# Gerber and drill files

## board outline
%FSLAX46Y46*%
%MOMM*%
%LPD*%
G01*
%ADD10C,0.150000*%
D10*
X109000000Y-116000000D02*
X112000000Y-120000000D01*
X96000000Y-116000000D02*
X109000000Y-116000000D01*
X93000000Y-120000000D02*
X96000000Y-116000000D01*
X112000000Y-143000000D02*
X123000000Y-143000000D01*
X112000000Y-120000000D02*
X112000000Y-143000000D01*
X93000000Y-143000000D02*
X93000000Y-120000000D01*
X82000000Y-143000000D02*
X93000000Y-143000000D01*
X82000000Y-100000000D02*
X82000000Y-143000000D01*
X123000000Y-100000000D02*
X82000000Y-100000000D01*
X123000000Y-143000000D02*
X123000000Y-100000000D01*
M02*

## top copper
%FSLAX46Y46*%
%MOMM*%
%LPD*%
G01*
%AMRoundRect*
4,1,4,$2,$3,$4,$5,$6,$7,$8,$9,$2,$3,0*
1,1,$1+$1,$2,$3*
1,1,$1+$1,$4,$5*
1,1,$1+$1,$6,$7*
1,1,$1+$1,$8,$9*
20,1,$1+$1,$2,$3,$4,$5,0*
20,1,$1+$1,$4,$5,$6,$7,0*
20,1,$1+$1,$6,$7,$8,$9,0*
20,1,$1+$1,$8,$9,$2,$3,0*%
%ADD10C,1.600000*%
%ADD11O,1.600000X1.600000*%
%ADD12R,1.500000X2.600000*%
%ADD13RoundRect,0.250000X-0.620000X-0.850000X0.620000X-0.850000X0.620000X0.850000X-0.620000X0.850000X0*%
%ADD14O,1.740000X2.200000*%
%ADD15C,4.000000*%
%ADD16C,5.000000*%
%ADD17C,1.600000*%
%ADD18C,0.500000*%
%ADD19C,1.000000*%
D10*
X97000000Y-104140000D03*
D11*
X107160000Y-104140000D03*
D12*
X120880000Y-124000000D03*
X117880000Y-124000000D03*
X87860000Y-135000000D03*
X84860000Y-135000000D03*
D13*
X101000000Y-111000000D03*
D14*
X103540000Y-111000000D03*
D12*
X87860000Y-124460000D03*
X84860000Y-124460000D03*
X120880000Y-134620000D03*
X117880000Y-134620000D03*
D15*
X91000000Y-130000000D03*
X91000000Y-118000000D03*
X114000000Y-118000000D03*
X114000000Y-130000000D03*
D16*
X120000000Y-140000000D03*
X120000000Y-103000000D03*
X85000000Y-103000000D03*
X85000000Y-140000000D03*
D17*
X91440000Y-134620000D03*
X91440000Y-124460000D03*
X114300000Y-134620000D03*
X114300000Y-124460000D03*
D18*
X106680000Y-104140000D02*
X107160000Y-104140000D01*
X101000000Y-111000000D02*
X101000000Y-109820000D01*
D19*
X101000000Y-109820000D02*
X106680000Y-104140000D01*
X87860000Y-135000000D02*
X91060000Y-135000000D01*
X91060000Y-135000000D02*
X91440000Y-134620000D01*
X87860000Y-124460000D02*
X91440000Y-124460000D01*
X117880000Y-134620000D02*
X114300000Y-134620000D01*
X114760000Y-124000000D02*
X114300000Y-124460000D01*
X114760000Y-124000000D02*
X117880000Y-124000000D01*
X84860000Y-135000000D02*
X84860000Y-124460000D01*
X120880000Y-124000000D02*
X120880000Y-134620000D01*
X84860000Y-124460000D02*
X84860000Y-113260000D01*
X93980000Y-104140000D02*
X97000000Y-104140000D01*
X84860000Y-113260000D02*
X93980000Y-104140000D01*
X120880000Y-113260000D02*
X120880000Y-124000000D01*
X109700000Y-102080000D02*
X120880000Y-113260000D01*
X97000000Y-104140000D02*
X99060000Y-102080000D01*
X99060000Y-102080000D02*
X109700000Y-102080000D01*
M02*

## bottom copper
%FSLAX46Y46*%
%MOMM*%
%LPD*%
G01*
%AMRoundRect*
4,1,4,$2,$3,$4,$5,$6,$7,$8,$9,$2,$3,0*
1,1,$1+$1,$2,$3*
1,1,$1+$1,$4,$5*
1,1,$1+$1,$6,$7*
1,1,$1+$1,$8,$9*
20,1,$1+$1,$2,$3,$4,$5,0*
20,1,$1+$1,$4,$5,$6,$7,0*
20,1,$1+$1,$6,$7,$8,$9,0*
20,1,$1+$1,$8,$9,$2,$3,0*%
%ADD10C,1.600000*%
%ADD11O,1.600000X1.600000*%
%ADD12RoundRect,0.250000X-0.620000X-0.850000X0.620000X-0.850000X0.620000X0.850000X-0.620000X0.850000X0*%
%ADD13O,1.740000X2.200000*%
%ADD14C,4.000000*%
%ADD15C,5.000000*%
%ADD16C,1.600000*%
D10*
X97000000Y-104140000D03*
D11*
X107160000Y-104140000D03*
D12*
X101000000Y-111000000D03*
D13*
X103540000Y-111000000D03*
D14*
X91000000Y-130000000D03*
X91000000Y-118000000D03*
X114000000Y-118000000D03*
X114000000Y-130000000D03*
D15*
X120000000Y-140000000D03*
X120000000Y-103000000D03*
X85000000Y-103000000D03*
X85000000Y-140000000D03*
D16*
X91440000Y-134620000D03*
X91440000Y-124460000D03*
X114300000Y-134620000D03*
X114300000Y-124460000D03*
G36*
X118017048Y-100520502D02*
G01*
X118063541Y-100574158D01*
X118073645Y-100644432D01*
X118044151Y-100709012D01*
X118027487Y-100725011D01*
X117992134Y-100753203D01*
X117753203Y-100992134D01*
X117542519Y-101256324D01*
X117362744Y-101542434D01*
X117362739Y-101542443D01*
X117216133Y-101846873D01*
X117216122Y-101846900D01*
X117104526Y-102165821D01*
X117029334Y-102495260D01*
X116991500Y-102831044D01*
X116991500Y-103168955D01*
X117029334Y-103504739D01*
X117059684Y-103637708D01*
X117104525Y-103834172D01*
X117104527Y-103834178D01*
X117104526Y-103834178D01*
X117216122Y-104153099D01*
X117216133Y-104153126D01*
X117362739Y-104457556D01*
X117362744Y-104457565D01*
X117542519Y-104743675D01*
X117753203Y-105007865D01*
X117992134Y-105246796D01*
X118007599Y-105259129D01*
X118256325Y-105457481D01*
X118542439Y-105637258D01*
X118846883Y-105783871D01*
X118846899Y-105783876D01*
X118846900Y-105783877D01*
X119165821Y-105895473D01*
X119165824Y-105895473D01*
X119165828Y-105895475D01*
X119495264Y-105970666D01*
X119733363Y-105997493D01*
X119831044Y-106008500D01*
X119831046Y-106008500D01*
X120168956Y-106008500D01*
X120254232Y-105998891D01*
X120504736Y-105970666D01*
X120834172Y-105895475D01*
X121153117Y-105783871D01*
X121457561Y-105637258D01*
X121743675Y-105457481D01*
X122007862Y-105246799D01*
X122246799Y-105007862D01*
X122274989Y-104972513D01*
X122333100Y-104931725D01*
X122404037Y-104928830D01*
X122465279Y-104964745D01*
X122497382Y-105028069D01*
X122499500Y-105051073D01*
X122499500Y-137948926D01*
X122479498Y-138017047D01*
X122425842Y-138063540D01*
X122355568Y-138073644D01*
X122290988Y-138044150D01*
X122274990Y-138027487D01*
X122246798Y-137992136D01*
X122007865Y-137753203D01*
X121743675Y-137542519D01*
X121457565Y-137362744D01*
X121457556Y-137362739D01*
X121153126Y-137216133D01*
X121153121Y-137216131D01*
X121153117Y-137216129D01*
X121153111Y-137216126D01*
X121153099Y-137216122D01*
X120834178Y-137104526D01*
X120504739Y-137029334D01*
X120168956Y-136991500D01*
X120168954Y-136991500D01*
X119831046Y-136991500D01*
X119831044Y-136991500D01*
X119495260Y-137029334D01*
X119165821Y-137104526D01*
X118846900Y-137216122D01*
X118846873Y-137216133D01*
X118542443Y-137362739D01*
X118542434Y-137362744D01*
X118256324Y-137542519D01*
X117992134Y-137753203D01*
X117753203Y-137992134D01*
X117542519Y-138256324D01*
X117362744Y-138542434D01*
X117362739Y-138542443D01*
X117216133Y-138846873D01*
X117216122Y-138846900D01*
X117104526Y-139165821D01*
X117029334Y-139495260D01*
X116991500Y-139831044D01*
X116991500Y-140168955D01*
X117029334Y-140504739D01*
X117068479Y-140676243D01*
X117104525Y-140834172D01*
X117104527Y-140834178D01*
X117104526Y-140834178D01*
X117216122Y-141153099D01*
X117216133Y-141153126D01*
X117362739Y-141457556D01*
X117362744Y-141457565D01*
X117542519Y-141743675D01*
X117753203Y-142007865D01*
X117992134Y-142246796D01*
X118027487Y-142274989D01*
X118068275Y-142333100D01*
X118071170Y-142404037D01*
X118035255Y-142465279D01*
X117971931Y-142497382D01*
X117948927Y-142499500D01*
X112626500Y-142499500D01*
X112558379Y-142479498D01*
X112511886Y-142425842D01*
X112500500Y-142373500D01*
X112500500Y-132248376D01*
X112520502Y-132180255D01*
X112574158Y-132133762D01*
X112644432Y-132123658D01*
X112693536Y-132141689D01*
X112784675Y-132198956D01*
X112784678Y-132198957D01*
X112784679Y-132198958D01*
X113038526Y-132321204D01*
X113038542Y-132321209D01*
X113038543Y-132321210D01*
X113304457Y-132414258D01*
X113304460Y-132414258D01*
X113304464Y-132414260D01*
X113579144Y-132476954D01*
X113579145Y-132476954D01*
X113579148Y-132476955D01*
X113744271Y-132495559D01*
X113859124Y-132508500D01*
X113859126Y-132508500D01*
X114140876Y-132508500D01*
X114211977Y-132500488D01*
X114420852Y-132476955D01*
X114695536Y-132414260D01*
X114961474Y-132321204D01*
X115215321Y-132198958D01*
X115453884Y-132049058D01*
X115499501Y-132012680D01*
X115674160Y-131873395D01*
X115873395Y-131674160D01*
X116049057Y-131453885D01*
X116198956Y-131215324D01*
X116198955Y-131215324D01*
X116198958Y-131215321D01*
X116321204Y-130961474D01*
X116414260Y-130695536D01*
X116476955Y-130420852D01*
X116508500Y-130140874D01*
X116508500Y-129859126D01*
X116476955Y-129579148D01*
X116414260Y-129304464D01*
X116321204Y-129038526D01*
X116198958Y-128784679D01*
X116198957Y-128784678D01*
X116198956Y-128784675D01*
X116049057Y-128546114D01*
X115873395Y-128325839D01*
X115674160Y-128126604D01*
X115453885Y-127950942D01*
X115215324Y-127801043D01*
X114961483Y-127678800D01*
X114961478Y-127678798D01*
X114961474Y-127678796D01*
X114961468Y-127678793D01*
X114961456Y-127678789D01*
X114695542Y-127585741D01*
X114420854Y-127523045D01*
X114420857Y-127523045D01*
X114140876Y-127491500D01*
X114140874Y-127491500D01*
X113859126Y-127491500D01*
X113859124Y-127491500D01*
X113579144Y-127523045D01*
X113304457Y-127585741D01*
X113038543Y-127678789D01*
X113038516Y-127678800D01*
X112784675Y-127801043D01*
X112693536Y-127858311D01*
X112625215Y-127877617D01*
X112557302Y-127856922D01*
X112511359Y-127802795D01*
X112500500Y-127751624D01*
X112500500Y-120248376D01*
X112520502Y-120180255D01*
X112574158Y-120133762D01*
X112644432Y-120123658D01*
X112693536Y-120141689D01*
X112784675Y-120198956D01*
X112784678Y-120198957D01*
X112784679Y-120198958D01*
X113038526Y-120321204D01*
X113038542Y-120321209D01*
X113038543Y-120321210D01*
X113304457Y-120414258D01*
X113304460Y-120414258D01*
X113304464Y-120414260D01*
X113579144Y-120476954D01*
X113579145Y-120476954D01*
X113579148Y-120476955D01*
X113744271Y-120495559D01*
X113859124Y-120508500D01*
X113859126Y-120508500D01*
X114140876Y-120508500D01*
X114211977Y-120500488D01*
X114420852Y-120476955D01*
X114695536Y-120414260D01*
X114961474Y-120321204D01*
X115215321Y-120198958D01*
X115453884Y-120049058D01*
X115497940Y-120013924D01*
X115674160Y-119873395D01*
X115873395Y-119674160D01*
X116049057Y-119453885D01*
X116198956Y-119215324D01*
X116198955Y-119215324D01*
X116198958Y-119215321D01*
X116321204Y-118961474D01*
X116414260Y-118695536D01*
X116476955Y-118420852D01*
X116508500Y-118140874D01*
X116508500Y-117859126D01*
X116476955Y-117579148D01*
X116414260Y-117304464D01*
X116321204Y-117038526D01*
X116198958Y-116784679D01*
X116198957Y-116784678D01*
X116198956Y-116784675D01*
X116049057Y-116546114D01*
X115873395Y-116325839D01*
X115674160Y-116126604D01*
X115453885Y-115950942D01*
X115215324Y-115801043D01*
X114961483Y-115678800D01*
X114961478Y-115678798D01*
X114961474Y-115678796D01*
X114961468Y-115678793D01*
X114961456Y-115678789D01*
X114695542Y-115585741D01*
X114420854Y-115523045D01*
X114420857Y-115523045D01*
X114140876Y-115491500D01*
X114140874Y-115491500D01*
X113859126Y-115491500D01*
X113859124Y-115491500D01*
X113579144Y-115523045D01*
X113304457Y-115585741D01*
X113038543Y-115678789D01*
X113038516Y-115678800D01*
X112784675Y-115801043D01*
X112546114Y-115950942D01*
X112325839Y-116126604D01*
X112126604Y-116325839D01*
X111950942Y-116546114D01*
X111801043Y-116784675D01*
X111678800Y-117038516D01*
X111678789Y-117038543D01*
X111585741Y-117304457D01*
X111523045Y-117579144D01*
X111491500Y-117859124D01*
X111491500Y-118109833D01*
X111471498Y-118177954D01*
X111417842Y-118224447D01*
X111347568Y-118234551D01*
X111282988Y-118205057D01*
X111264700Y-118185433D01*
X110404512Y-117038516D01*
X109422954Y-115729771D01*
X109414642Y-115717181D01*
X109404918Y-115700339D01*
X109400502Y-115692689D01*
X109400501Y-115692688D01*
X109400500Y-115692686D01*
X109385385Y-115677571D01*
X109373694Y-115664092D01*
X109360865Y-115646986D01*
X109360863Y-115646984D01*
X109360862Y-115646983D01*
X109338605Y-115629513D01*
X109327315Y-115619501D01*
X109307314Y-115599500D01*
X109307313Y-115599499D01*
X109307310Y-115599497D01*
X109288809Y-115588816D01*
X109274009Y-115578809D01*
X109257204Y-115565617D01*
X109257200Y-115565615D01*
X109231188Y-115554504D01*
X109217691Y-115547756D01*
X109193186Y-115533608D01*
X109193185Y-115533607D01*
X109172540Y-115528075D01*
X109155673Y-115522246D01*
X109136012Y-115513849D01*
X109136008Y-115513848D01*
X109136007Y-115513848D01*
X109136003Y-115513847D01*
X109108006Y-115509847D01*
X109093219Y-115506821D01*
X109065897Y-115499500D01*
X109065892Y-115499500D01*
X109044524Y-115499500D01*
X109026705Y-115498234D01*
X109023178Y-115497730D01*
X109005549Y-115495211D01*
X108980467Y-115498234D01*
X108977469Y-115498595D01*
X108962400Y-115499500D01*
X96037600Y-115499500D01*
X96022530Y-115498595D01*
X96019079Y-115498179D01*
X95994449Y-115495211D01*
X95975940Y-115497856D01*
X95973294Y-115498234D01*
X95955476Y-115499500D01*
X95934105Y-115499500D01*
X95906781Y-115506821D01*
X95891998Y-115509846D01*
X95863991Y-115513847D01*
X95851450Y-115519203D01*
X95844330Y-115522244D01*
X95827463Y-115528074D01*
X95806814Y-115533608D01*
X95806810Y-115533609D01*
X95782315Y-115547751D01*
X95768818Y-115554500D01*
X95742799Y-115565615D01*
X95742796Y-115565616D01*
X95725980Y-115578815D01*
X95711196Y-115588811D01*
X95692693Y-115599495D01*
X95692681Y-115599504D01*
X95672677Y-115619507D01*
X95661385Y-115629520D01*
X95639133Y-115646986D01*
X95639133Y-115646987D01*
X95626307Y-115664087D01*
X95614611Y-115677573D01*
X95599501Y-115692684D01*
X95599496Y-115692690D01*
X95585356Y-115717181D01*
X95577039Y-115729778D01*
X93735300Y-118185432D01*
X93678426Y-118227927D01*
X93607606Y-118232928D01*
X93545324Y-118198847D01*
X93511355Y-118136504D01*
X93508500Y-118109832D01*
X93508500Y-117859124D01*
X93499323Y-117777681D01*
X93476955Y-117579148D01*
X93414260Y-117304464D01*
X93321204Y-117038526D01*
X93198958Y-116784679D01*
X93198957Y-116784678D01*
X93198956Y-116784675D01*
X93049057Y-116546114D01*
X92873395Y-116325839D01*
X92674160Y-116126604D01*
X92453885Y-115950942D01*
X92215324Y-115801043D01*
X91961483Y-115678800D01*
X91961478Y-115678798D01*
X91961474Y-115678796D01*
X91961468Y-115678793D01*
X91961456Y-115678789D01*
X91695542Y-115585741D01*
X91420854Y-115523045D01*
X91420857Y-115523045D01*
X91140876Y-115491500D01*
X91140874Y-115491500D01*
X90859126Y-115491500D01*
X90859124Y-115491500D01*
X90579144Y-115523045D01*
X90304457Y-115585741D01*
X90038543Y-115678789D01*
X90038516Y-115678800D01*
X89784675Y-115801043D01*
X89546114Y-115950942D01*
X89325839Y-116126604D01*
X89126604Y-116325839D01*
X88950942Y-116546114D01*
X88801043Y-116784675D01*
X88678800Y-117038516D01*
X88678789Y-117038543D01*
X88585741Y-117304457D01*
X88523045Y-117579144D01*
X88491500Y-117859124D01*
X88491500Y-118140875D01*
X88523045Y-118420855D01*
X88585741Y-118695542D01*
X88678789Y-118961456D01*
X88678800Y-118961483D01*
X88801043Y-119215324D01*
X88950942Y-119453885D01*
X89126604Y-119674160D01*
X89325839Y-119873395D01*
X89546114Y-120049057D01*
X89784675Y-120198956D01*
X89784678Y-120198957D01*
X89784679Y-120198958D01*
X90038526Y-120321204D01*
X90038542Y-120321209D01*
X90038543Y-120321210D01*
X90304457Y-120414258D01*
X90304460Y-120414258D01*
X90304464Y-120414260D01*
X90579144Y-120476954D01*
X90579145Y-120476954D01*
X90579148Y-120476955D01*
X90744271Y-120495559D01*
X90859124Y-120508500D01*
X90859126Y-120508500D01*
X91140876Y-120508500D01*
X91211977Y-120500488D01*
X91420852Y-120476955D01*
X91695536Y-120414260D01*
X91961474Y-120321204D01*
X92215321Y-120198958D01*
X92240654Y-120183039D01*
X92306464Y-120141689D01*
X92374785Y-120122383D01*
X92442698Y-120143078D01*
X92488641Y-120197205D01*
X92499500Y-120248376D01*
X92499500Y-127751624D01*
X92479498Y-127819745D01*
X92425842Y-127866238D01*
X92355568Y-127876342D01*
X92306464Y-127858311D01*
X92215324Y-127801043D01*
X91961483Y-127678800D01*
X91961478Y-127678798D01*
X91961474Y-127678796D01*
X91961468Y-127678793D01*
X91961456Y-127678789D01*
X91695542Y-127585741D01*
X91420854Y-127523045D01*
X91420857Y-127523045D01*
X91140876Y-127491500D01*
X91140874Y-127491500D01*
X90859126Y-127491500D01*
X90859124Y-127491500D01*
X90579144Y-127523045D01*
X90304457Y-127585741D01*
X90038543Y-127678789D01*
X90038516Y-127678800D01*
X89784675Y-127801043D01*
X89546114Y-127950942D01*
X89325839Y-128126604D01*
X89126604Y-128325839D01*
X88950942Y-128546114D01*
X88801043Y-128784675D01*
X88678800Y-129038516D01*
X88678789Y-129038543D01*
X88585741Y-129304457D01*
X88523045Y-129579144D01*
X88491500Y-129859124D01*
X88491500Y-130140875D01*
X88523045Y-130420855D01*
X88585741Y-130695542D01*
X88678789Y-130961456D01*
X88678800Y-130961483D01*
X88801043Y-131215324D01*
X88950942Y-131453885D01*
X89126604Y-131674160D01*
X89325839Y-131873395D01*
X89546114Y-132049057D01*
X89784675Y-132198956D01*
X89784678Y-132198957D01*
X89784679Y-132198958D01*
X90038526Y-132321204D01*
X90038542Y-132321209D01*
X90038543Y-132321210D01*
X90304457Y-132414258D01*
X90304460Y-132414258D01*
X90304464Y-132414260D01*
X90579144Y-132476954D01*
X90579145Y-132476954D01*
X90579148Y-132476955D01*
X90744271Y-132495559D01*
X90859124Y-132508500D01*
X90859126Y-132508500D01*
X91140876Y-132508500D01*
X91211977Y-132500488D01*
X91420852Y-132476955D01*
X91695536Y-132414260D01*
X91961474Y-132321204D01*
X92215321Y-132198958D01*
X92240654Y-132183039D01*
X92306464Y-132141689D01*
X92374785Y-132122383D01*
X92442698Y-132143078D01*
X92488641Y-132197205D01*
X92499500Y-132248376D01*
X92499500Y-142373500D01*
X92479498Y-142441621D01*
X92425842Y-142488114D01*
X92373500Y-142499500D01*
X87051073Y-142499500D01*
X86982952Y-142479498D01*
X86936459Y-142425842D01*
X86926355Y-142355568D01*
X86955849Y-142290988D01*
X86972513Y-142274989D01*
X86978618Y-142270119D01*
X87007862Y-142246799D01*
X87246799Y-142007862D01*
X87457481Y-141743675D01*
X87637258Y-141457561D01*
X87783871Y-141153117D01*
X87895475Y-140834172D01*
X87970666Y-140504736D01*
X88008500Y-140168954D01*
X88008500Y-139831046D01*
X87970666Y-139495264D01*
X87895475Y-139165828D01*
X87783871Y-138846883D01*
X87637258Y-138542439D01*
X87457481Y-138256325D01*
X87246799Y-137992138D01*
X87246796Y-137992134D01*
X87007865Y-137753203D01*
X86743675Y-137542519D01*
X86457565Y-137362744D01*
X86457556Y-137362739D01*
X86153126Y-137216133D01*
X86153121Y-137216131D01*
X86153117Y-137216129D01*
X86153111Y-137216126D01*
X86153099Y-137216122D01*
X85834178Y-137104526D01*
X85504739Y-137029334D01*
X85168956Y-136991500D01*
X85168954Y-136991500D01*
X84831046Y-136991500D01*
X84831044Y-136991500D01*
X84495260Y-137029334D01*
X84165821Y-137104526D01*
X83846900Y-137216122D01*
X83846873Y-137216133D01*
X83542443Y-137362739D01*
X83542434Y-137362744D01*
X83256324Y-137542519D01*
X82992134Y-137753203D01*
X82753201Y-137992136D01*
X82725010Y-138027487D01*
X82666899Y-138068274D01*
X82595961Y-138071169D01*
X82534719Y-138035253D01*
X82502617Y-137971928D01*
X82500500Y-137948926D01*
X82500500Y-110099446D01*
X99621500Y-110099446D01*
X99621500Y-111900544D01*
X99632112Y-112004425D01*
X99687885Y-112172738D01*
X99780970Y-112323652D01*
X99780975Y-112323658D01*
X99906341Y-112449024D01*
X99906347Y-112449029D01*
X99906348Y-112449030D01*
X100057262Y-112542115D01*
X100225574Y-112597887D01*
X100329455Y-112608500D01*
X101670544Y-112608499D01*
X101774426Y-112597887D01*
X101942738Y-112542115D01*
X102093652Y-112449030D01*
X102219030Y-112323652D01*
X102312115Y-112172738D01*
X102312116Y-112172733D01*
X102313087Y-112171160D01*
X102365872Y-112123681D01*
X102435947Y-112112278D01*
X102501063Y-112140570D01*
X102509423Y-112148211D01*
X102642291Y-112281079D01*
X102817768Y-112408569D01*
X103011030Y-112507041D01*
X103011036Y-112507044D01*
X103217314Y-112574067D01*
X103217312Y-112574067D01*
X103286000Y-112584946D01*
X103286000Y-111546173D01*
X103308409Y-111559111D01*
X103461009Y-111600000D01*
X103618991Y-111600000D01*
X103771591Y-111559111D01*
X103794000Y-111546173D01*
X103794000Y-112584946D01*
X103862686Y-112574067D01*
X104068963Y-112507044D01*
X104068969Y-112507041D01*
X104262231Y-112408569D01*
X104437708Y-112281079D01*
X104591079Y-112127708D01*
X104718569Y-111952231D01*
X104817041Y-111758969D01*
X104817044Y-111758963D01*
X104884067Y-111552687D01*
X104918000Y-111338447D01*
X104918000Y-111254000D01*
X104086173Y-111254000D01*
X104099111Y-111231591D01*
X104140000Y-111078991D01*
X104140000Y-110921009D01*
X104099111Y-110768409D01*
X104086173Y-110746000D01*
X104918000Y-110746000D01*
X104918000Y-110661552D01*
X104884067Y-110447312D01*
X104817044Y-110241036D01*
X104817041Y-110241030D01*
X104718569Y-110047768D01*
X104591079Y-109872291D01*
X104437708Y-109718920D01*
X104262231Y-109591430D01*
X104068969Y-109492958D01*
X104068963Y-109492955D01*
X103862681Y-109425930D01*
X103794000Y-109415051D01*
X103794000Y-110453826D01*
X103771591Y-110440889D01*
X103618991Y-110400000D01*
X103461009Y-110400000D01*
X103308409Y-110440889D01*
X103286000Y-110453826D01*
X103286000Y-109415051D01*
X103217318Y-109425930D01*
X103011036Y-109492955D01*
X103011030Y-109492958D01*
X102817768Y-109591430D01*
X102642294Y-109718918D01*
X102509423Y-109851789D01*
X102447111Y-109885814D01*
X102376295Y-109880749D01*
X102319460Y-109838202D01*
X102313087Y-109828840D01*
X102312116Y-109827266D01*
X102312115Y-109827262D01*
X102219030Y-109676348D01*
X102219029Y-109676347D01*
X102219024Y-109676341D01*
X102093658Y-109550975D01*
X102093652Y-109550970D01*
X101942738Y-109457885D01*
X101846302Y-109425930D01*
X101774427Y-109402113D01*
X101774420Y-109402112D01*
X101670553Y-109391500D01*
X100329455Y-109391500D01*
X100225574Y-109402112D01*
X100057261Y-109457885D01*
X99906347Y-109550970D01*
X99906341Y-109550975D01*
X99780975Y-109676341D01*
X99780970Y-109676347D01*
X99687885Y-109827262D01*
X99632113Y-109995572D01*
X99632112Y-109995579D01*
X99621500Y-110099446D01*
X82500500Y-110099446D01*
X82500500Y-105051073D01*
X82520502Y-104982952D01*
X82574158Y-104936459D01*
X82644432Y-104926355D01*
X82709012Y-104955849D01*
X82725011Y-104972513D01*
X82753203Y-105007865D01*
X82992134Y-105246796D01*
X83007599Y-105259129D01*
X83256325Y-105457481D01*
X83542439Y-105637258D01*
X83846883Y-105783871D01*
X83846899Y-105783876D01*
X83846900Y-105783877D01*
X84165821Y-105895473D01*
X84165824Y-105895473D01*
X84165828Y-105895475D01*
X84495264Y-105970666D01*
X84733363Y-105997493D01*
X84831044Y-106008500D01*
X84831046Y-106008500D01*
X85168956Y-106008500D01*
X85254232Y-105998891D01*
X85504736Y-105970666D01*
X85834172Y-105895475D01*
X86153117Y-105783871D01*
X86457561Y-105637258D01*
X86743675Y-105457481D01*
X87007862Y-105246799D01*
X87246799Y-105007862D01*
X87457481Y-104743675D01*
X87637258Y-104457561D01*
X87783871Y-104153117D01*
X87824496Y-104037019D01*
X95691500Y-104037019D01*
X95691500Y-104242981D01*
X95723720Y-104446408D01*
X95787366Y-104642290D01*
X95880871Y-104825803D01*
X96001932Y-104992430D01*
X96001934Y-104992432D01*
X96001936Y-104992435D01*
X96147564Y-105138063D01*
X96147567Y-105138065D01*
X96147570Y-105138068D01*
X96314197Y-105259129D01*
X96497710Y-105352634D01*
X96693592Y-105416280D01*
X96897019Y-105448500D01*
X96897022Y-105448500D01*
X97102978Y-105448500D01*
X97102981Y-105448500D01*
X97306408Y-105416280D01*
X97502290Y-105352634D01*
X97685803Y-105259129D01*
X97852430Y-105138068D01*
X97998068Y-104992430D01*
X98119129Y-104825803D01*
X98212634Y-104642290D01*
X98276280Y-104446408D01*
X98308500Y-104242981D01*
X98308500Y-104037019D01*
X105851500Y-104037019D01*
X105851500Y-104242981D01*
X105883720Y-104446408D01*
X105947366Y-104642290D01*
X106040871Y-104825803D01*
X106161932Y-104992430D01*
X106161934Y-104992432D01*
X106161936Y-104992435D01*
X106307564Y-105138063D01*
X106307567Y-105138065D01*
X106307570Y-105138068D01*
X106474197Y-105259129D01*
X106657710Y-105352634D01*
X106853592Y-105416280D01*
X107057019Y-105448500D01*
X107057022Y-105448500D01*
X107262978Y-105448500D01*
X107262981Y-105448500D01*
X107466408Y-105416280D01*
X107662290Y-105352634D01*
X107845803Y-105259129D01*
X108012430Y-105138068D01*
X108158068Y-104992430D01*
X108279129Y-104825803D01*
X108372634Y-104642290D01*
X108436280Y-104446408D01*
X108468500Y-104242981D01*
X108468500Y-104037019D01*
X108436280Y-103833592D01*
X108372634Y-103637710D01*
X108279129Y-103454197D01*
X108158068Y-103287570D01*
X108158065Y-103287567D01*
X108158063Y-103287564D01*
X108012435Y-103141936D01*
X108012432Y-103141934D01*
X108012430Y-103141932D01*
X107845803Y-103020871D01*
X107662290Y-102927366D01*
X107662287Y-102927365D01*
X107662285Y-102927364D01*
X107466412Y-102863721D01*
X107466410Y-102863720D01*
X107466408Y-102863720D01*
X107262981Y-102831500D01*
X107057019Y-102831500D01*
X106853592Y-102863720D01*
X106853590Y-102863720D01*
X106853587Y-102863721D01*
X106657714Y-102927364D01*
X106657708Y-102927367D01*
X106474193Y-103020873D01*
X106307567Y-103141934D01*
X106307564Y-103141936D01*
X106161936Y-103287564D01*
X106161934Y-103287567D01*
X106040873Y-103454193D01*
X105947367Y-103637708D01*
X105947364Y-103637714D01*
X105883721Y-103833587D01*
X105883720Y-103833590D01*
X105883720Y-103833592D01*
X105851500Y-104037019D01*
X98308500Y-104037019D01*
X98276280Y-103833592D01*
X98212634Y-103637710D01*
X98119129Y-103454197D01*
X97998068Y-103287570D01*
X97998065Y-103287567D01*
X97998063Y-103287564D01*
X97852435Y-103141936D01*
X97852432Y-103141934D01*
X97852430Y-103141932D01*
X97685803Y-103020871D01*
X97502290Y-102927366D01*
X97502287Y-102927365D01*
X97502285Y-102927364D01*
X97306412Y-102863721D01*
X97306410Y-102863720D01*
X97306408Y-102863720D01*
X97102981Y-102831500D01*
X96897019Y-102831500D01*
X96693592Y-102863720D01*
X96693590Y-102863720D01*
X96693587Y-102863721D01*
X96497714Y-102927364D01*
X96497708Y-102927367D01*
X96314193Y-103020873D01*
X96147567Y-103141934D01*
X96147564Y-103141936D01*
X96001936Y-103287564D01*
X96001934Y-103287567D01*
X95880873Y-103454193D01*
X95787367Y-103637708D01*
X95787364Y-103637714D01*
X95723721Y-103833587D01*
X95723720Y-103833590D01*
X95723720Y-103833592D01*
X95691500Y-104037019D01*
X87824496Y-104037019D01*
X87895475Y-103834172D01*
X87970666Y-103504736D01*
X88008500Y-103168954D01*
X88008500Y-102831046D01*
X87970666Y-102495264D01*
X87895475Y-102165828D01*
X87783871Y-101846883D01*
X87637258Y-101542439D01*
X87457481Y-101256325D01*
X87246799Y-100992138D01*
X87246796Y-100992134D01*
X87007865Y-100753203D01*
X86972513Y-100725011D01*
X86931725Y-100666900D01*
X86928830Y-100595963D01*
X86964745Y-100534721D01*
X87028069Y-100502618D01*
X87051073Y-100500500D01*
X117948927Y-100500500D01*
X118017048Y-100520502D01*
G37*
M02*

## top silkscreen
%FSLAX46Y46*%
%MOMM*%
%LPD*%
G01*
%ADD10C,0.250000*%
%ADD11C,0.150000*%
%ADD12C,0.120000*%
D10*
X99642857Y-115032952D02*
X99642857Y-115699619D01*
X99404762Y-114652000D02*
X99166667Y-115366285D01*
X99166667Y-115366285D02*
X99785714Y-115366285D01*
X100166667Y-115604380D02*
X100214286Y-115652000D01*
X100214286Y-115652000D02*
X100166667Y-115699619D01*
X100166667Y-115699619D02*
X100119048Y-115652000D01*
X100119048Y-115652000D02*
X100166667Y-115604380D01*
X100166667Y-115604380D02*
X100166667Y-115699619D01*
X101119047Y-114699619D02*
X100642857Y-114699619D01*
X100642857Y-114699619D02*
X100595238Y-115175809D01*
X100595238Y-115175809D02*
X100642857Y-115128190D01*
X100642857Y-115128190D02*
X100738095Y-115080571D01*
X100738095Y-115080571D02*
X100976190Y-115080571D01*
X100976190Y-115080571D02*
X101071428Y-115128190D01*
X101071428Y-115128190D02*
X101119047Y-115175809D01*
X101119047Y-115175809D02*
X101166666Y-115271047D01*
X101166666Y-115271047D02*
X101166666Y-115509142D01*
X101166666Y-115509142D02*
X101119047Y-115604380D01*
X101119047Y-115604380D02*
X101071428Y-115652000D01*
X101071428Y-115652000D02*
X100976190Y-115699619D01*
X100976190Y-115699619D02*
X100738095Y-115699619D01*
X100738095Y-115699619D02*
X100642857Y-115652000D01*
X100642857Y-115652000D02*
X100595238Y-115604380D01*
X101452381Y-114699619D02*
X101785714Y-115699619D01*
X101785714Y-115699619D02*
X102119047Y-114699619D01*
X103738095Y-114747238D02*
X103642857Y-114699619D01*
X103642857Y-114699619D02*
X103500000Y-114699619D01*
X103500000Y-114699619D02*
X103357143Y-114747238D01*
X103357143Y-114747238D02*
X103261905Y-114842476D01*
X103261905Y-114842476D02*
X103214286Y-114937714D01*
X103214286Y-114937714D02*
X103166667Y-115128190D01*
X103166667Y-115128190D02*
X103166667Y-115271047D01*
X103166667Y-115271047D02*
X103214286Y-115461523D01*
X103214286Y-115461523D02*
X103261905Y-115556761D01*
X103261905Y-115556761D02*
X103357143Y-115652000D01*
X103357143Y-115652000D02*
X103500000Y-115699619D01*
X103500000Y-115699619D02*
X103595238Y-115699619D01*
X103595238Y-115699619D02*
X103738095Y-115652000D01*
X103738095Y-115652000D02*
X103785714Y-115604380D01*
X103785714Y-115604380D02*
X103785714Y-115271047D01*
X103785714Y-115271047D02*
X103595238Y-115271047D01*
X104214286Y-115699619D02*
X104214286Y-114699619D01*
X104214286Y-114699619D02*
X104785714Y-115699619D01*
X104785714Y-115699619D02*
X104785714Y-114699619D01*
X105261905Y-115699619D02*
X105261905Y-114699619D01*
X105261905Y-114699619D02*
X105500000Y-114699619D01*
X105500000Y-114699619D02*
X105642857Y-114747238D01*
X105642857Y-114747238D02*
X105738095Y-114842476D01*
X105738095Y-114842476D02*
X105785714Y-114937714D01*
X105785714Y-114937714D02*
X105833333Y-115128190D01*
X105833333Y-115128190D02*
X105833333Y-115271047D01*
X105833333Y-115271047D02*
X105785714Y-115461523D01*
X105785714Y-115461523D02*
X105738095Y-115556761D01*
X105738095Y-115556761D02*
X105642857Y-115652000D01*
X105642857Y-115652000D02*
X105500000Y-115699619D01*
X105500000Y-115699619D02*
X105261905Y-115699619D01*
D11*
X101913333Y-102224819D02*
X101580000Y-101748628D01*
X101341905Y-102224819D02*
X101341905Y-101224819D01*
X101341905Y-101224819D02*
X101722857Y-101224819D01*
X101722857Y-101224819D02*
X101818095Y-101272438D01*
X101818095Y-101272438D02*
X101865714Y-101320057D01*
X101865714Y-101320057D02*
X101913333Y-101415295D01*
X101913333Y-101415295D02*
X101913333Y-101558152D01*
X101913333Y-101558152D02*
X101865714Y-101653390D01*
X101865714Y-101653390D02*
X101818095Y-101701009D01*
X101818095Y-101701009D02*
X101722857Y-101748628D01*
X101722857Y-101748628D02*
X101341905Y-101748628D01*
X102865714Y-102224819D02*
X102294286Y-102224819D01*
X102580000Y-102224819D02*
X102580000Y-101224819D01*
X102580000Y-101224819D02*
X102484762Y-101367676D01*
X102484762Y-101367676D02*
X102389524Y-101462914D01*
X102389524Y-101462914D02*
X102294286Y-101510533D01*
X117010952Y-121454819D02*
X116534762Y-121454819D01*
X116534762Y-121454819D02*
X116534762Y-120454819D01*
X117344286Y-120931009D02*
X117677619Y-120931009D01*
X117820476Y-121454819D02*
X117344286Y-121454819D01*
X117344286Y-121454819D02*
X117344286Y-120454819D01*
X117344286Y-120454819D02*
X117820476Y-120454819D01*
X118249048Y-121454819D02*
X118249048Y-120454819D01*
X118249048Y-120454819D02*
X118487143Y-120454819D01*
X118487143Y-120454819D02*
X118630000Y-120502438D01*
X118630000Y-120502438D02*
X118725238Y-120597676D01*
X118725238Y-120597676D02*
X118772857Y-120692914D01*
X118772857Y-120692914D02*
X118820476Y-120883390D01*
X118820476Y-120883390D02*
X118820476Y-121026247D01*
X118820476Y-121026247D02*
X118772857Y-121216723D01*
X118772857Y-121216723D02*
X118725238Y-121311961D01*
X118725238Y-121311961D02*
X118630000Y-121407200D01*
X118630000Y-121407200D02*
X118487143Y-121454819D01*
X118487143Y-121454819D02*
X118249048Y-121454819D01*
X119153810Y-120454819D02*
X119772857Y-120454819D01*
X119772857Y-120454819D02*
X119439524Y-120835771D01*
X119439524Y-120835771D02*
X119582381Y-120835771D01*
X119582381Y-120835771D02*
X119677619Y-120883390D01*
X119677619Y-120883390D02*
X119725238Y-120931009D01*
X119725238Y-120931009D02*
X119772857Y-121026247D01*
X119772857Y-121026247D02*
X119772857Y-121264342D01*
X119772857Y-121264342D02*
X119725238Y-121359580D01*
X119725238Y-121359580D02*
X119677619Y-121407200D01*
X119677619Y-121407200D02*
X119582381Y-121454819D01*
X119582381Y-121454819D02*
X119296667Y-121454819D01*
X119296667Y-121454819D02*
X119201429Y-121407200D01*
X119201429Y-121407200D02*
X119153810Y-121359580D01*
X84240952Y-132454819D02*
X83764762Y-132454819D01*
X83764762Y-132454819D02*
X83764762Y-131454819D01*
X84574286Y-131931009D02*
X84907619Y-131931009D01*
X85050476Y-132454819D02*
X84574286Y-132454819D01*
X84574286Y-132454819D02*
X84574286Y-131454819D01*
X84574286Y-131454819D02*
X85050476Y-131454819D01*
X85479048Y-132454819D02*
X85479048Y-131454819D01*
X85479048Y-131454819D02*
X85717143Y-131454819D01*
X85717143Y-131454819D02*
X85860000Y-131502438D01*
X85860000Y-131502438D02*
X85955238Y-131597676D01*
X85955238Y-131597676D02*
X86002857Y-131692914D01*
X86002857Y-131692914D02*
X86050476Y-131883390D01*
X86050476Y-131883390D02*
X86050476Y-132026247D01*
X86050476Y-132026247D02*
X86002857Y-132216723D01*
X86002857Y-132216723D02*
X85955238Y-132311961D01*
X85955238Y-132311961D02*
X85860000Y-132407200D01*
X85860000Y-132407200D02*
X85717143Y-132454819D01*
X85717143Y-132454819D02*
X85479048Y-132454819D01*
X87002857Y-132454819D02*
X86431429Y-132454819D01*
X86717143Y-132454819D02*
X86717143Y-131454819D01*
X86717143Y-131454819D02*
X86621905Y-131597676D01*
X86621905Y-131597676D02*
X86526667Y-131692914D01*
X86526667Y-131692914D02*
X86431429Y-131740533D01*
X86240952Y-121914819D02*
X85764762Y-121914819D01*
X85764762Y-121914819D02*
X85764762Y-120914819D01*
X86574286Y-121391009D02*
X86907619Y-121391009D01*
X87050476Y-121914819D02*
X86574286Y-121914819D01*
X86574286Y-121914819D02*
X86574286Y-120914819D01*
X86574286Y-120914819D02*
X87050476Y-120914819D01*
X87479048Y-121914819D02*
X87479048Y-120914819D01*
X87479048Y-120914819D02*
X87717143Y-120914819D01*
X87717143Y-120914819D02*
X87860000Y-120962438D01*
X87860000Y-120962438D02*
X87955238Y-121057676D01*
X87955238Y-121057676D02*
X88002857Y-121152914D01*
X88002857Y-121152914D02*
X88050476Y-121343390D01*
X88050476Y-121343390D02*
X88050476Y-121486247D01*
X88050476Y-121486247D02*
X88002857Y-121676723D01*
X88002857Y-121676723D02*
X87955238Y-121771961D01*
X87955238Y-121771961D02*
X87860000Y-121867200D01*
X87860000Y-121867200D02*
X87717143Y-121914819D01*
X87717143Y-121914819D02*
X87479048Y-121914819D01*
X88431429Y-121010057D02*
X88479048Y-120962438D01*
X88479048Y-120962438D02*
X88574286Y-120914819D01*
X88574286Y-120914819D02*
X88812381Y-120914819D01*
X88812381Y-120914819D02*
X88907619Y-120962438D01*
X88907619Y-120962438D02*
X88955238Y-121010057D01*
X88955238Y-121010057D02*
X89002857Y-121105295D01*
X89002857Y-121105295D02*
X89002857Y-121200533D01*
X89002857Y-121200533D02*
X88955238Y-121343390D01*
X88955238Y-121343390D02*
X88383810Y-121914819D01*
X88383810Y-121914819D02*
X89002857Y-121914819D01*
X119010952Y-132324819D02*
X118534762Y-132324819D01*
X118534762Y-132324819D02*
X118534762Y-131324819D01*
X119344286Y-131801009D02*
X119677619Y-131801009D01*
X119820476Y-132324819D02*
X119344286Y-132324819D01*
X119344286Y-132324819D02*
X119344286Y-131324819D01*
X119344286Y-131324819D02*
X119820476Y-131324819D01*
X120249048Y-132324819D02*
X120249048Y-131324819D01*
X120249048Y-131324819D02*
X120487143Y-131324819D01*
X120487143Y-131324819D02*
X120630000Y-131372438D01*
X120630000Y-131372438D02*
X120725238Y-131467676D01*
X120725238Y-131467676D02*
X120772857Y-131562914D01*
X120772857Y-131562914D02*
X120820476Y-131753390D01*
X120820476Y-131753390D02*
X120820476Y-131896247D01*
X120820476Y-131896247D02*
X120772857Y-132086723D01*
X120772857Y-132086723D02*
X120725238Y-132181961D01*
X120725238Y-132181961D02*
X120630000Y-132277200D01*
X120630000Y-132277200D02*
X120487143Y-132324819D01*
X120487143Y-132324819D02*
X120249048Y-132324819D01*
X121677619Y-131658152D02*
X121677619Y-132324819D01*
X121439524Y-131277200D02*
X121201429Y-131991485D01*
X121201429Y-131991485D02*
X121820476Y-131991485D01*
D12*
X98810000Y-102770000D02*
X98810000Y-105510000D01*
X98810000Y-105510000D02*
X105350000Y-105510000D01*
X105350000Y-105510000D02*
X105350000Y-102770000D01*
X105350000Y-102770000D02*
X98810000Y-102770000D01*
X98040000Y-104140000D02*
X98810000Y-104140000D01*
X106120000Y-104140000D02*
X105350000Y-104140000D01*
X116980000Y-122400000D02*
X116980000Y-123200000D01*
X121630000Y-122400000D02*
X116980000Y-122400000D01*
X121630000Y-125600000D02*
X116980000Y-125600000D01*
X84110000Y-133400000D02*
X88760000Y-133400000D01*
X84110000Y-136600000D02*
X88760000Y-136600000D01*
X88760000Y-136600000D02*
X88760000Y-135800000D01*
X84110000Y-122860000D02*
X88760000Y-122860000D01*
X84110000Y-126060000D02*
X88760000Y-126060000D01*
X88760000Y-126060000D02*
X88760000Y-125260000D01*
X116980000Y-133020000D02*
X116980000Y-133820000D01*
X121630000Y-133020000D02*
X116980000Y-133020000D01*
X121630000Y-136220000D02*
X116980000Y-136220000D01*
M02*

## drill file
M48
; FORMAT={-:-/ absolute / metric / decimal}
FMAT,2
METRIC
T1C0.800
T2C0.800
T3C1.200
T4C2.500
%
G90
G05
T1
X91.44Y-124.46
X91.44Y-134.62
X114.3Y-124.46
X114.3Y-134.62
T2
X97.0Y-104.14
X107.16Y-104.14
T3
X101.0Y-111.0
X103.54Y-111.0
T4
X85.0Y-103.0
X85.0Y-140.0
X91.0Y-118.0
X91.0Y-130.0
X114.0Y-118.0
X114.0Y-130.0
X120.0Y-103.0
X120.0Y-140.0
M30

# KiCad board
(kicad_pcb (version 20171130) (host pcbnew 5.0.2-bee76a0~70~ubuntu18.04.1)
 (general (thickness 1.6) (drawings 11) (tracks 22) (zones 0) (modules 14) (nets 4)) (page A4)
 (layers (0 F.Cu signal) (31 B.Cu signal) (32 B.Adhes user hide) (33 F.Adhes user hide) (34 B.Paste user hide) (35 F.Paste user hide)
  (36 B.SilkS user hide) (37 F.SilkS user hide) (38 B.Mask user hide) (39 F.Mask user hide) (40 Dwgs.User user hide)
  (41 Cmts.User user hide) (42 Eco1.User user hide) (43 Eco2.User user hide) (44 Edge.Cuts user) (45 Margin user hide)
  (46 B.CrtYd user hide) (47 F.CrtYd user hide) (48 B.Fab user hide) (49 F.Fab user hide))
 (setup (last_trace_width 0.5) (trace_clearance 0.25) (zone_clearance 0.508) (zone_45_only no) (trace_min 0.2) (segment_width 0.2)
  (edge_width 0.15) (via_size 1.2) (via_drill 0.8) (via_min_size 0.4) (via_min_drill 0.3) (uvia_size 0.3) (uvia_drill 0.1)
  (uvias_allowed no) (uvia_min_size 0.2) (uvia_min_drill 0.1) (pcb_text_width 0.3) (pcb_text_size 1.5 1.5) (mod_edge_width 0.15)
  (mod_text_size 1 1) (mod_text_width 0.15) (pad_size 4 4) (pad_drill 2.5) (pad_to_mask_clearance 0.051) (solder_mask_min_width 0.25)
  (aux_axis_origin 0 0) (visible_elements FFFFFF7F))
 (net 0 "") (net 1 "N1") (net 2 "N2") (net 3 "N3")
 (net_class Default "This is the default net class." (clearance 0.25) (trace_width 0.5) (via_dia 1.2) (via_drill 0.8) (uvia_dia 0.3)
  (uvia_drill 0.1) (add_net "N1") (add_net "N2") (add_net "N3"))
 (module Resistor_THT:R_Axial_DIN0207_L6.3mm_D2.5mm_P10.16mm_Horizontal (layer F.Cu) (at 97 104.14)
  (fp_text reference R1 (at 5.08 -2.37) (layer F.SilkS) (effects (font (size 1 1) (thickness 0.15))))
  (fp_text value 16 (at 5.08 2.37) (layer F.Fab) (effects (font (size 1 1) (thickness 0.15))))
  (fp_line (start 1.81 -1.37) (end 1.81 1.37) (layer F.SilkS) (width 0.12))
  (fp_line (start 1.81 1.37) (end 8.35 1.37) (layer F.SilkS) (width 0.12))
  (fp_line (start 8.35 1.37) (end 8.35 -1.37) (layer F.SilkS) (width 0.12))
  (fp_line (start 8.35 -1.37) (end 1.81 -1.37) (layer F.SilkS) (width 0.12))
  (fp_line (start 1.04 0) (end 1.81 0) (layer F.SilkS) (width 0.12))
  (fp_line (start 9.12 0) (end 8.35 0) (layer F.SilkS) (width 0.12))
  (pad 1 thru_hole circle (at 0 0) (size 1.6 1.6) (drill 0.8) (layers *.Cu *.Mask) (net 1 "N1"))
  (pad 2 thru_hole oval (at 10.16 0) (size 1.6 1.6) (drill 0.8) (layers *.Cu *.Mask) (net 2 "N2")))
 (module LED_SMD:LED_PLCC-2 (layer F.Cu) (at 119.38 124)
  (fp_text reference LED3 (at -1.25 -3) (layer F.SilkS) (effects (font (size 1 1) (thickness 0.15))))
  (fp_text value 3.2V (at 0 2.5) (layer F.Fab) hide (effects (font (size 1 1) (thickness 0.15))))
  (fp_line (start -2.4 -1.6) (end -2.4 -0.8) (layer F.SilkS) (width 0.12))
  (fp_line (start 2.25 -1.6) (end -2.4 -1.6) (layer F.SilkS) (width 0.12))
  (fp_line (start 2.25 1.6) (end -2.4 1.6) (layer F.SilkS) (width 0.12))
  (pad 2 smd rect (at 1.5 0) (size 1.5 2.6) (layers F.Cu F.Paste F.Mask) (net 1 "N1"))
  (pad 1 smd rect (at -1.5 0) (size 1.5 2.6) (layers F.Cu F.Paste F.Mask) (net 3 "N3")))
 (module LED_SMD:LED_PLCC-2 (layer F.Cu) (at 86.36 135 180)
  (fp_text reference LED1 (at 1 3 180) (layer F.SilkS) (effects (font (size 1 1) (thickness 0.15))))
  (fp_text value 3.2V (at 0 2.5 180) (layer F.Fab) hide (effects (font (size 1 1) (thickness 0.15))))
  (fp_line (start 2.25 1.6) (end -2.4 1.6) (layer F.SilkS) (width 0.12))
  (fp_line (start 2.25 -1.6) (end -2.4 -1.6) (layer F.SilkS) (width 0.12))
  (fp_line (start -2.4 -1.6) (end -2.4 -0.8) (layer F.SilkS) (width 0.12))
  (pad 1 smd rect (at -1.5 0 180) (size 1.5 2.6) (layers F.Cu F.Paste F.Mask) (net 3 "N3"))
  (pad 2 smd rect (at 1.5 0 180) (size 1.5 2.6) (layers F.Cu F.Paste F.Mask) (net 1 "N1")))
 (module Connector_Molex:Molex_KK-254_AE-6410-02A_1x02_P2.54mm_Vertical (layer B.Cu) (at 101 111)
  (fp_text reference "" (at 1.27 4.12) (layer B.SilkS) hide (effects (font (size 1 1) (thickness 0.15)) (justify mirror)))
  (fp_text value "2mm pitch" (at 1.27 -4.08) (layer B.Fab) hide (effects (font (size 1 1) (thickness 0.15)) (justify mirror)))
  (pad 1 thru_hole roundrect (at 0 0) (size 1.74 2.2) (drill 1.2) (layers *.Cu *.Mask) (roundrect_rratio 0.143678) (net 2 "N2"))
  (pad 2 thru_hole oval (at 2.54 0) (size 1.74 2.2) (drill 1.2) (layers *.Cu *.Mask) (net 3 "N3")))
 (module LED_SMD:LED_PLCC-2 (layer F.Cu) (at 86.36 124.46 180)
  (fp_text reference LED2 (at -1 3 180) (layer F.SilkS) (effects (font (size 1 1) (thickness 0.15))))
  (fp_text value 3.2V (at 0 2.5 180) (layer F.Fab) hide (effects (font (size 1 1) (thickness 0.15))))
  (fp_line (start 2.25 1.6) (end -2.4 1.6) (layer F.SilkS) (width 0.12))
  (fp_line (start 2.25 -1.6) (end -2.4 -1.6) (layer F.SilkS) (width 0.12))
  (fp_line (start -2.4 -1.6) (end -2.4 -0.8) (layer F.SilkS) (width 0.12))
  (pad 1 smd rect (at -1.5 0 180) (size 1.5 2.6) (layers F.Cu F.Paste F.Mask) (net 3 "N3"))
  (pad 2 smd rect (at 1.5 0 180) (size 1.5 2.6) (layers F.Cu F.Paste F.Mask) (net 1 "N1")))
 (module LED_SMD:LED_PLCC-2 (layer F.Cu) (at 119.38 134.62)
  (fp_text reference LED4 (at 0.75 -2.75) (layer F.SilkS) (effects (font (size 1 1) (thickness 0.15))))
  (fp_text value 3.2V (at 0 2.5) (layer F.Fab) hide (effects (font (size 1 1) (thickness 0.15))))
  (fp_line (start -2.4 -1.6) (end -2.4 -0.8) (layer F.SilkS) (width 0.12))
  (fp_line (start 2.25 -1.6) (end -2.4 -1.6) (layer F.SilkS) (width 0.12))
  (fp_line (start 2.25 1.6) (end -2.4 1.6) (layer F.SilkS) (width 0.12))
  (pad 2 smd rect (at 1.5 0) (size 1.5 2.6) (layers F.Cu F.Paste F.Mask) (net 1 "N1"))
  (pad 1 smd rect (at -1.5 0) (size 1.5 2.6) (layers F.Cu F.Paste F.Mask) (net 3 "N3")))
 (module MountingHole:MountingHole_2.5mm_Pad (layer F.Cu) (at 91 130)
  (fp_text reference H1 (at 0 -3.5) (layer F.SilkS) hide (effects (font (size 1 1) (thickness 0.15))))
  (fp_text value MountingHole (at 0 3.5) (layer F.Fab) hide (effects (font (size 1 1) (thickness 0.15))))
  (pad 1 thru_hole circle (at 0 0) (size 4 4) (drill 2.5) (layers *.Cu *.Mask)))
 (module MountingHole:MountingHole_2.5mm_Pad (layer F.Cu) (at 91 118)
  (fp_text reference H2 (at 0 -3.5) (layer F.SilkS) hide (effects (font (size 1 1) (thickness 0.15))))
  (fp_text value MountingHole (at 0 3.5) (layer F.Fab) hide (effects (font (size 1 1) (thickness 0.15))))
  (pad 1 thru_hole circle (at 0 0) (size 4 4) (drill 2.5) (layers *.Cu *.Mask)))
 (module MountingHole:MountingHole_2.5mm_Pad (layer F.Cu) (at 114 118)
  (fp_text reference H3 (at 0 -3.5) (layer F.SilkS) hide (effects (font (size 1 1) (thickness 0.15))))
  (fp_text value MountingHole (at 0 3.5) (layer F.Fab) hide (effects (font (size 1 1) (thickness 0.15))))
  (pad 1 thru_hole circle (at 0 0) (size 4 4) (drill 2.5) (layers *.Cu *.Mask)))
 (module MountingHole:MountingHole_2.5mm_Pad (layer F.Cu) (at 114 130)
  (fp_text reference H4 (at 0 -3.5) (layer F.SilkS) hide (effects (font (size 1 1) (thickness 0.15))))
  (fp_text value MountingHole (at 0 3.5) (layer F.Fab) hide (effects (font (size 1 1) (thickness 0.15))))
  (pad 1 thru_hole circle (at 0 0) (size 4 4) (drill 2.5) (layers *.Cu *.Mask)))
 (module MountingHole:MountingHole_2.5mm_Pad (layer F.Cu) (at 120 140)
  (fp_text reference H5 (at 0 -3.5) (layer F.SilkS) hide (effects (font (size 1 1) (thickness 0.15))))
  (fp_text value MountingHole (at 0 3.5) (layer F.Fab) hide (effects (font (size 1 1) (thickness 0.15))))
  (pad 1 thru_hole circle (at 0 0) (size 5 5) (drill 2.5) (layers *.Cu *.Mask)))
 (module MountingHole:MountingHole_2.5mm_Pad (layer F.Cu) (at 120 103)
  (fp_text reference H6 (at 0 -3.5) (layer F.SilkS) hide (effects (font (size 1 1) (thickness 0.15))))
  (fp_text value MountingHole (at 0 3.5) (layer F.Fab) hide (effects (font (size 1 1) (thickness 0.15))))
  (pad 1 thru_hole circle (at 0 0) (size 5 5) (drill 2.5) (layers *.Cu *.Mask)))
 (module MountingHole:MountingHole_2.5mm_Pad (layer F.Cu) (at 85 103)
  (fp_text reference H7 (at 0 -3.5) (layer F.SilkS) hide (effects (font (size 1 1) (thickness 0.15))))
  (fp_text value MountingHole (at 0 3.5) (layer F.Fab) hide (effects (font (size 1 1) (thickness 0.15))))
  (pad 1 thru_hole circle (at 0 0) (size 5 5) (drill 2.5) (layers *.Cu *.Mask)))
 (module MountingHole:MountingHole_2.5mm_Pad (layer F.Cu) (at 85 140)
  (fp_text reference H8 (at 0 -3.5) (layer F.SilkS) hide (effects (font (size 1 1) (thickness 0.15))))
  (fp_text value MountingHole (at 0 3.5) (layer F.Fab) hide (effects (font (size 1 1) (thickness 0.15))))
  (pad 1 thru_hole circle (at 0 0) (size 5 5) (drill 2.5) (layers *.Cu *.Mask)))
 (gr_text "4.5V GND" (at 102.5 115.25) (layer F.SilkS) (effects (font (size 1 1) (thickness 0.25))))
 (gr_line (start 109 116) (end 112 120) (layer Edge.Cuts) (width 0.15))
 (gr_line (start 96 116) (end 109 116) (layer Edge.Cuts) (width 0.15))
 (gr_line (start 93 120) (end 96 116) (layer Edge.Cuts) (width 0.15))
 (gr_line (start 112 143) (end 123 143) (layer Edge.Cuts) (width 0.15))
 (gr_line (start 112 120) (end 112 143) (layer Edge.Cuts) (width 0.15))
 (gr_line (start 93 143) (end 93 120) (layer Edge.Cuts) (width 0.15))
 (gr_line (start 82 143) (end 93 143) (layer Edge.Cuts) (width 0.15))
 (gr_line (start 82 100) (end 82 143) (layer Edge.Cuts) (width 0.15))
 (gr_line (start 123 100) (end 82 100) (layer Edge.Cuts) (width 0.15))
 (gr_line (start 123 143) (end 123 100) (layer Edge.Cuts) (width 0.15))
 (segment (start 106.68 104.14) (end 107.16 104.14) (width 0.5) (layer F.Cu) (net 2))
 (segment (start 101 111) (end 101 109.82) (width 0.5) (layer F.Cu) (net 2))
 (segment (start 101 109.82) (end 106.68 104.14) (width 1) (layer F.Cu) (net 2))
 (segment (start 87.86 135) (end 91.06 135) (width 1) (layer F.Cu) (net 3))
 (via (at 91.44 134.62) (size 1.6) (drill 0.8) (layers F.Cu B.Cu) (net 3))
 (segment (start 91.06 135) (end 91.44 134.62) (width 1) (layer F.Cu) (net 3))
 (via (at 91.44 124.46) (size 1.6) (drill 0.8) (layers F.Cu B.Cu) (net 3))
 (segment (start 87.86 124.46) (end 91.44 124.46) (width 1) (layer F.Cu) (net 3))
 (segment (start 117.88 134.62) (end 114.3 134.62) (width 1) (layer F.Cu) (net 3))
 (via (at 114.3 134.62) (size 1.6) (drill 0.8) (layers F.Cu B.Cu) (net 3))
 (via (at 114.3 124.46) (size 1.6) (drill 0.8) (layers F.Cu B.Cu) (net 3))
 (segment (start 114.76 124) (end 114.3 124.46) (width 1) (layer F.Cu) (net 3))
 (segment (start 114.76 124) (end 117.88 124) (width 1) (layer F.Cu) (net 3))
 (segment (start 84.86 135) (end 84.86 124.46) (width 1) (layer F.Cu) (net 1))
 (segment (start 120.88 124) (end 120.88 134.62) (width 1) (layer F.Cu) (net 1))
 (segment (start 84.86 124.46) (end 84.86 113.26) (width 1) (layer F.Cu) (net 1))
 (segment (start 93.98 104.14) (end 97 104.14) (width 1) (layer F.Cu) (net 1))
 (segment (start 84.86 113.26) (end 93.98 104.14) (width 1) (layer F.Cu) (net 1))
 (segment (start 120.88 113.26) (end 120.88 124) (width 1) (layer F.Cu) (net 1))
 (segment (start 109.7 102.08) (end 120.88 113.26) (width 1) (layer F.Cu) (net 1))
 (segment (start 97 104.14) (end 99.06 102.08) (width 1) (layer F.Cu) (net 1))
 (segment (start 99.06 102.08) (end 109.7 102.08) (width 1) (layer F.Cu) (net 1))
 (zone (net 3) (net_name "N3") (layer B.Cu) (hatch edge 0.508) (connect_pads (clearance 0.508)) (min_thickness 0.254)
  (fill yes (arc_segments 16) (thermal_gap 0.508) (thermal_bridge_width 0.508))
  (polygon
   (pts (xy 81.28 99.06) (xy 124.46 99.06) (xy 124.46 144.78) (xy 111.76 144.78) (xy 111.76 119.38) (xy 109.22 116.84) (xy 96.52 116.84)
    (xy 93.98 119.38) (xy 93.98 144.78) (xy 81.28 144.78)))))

